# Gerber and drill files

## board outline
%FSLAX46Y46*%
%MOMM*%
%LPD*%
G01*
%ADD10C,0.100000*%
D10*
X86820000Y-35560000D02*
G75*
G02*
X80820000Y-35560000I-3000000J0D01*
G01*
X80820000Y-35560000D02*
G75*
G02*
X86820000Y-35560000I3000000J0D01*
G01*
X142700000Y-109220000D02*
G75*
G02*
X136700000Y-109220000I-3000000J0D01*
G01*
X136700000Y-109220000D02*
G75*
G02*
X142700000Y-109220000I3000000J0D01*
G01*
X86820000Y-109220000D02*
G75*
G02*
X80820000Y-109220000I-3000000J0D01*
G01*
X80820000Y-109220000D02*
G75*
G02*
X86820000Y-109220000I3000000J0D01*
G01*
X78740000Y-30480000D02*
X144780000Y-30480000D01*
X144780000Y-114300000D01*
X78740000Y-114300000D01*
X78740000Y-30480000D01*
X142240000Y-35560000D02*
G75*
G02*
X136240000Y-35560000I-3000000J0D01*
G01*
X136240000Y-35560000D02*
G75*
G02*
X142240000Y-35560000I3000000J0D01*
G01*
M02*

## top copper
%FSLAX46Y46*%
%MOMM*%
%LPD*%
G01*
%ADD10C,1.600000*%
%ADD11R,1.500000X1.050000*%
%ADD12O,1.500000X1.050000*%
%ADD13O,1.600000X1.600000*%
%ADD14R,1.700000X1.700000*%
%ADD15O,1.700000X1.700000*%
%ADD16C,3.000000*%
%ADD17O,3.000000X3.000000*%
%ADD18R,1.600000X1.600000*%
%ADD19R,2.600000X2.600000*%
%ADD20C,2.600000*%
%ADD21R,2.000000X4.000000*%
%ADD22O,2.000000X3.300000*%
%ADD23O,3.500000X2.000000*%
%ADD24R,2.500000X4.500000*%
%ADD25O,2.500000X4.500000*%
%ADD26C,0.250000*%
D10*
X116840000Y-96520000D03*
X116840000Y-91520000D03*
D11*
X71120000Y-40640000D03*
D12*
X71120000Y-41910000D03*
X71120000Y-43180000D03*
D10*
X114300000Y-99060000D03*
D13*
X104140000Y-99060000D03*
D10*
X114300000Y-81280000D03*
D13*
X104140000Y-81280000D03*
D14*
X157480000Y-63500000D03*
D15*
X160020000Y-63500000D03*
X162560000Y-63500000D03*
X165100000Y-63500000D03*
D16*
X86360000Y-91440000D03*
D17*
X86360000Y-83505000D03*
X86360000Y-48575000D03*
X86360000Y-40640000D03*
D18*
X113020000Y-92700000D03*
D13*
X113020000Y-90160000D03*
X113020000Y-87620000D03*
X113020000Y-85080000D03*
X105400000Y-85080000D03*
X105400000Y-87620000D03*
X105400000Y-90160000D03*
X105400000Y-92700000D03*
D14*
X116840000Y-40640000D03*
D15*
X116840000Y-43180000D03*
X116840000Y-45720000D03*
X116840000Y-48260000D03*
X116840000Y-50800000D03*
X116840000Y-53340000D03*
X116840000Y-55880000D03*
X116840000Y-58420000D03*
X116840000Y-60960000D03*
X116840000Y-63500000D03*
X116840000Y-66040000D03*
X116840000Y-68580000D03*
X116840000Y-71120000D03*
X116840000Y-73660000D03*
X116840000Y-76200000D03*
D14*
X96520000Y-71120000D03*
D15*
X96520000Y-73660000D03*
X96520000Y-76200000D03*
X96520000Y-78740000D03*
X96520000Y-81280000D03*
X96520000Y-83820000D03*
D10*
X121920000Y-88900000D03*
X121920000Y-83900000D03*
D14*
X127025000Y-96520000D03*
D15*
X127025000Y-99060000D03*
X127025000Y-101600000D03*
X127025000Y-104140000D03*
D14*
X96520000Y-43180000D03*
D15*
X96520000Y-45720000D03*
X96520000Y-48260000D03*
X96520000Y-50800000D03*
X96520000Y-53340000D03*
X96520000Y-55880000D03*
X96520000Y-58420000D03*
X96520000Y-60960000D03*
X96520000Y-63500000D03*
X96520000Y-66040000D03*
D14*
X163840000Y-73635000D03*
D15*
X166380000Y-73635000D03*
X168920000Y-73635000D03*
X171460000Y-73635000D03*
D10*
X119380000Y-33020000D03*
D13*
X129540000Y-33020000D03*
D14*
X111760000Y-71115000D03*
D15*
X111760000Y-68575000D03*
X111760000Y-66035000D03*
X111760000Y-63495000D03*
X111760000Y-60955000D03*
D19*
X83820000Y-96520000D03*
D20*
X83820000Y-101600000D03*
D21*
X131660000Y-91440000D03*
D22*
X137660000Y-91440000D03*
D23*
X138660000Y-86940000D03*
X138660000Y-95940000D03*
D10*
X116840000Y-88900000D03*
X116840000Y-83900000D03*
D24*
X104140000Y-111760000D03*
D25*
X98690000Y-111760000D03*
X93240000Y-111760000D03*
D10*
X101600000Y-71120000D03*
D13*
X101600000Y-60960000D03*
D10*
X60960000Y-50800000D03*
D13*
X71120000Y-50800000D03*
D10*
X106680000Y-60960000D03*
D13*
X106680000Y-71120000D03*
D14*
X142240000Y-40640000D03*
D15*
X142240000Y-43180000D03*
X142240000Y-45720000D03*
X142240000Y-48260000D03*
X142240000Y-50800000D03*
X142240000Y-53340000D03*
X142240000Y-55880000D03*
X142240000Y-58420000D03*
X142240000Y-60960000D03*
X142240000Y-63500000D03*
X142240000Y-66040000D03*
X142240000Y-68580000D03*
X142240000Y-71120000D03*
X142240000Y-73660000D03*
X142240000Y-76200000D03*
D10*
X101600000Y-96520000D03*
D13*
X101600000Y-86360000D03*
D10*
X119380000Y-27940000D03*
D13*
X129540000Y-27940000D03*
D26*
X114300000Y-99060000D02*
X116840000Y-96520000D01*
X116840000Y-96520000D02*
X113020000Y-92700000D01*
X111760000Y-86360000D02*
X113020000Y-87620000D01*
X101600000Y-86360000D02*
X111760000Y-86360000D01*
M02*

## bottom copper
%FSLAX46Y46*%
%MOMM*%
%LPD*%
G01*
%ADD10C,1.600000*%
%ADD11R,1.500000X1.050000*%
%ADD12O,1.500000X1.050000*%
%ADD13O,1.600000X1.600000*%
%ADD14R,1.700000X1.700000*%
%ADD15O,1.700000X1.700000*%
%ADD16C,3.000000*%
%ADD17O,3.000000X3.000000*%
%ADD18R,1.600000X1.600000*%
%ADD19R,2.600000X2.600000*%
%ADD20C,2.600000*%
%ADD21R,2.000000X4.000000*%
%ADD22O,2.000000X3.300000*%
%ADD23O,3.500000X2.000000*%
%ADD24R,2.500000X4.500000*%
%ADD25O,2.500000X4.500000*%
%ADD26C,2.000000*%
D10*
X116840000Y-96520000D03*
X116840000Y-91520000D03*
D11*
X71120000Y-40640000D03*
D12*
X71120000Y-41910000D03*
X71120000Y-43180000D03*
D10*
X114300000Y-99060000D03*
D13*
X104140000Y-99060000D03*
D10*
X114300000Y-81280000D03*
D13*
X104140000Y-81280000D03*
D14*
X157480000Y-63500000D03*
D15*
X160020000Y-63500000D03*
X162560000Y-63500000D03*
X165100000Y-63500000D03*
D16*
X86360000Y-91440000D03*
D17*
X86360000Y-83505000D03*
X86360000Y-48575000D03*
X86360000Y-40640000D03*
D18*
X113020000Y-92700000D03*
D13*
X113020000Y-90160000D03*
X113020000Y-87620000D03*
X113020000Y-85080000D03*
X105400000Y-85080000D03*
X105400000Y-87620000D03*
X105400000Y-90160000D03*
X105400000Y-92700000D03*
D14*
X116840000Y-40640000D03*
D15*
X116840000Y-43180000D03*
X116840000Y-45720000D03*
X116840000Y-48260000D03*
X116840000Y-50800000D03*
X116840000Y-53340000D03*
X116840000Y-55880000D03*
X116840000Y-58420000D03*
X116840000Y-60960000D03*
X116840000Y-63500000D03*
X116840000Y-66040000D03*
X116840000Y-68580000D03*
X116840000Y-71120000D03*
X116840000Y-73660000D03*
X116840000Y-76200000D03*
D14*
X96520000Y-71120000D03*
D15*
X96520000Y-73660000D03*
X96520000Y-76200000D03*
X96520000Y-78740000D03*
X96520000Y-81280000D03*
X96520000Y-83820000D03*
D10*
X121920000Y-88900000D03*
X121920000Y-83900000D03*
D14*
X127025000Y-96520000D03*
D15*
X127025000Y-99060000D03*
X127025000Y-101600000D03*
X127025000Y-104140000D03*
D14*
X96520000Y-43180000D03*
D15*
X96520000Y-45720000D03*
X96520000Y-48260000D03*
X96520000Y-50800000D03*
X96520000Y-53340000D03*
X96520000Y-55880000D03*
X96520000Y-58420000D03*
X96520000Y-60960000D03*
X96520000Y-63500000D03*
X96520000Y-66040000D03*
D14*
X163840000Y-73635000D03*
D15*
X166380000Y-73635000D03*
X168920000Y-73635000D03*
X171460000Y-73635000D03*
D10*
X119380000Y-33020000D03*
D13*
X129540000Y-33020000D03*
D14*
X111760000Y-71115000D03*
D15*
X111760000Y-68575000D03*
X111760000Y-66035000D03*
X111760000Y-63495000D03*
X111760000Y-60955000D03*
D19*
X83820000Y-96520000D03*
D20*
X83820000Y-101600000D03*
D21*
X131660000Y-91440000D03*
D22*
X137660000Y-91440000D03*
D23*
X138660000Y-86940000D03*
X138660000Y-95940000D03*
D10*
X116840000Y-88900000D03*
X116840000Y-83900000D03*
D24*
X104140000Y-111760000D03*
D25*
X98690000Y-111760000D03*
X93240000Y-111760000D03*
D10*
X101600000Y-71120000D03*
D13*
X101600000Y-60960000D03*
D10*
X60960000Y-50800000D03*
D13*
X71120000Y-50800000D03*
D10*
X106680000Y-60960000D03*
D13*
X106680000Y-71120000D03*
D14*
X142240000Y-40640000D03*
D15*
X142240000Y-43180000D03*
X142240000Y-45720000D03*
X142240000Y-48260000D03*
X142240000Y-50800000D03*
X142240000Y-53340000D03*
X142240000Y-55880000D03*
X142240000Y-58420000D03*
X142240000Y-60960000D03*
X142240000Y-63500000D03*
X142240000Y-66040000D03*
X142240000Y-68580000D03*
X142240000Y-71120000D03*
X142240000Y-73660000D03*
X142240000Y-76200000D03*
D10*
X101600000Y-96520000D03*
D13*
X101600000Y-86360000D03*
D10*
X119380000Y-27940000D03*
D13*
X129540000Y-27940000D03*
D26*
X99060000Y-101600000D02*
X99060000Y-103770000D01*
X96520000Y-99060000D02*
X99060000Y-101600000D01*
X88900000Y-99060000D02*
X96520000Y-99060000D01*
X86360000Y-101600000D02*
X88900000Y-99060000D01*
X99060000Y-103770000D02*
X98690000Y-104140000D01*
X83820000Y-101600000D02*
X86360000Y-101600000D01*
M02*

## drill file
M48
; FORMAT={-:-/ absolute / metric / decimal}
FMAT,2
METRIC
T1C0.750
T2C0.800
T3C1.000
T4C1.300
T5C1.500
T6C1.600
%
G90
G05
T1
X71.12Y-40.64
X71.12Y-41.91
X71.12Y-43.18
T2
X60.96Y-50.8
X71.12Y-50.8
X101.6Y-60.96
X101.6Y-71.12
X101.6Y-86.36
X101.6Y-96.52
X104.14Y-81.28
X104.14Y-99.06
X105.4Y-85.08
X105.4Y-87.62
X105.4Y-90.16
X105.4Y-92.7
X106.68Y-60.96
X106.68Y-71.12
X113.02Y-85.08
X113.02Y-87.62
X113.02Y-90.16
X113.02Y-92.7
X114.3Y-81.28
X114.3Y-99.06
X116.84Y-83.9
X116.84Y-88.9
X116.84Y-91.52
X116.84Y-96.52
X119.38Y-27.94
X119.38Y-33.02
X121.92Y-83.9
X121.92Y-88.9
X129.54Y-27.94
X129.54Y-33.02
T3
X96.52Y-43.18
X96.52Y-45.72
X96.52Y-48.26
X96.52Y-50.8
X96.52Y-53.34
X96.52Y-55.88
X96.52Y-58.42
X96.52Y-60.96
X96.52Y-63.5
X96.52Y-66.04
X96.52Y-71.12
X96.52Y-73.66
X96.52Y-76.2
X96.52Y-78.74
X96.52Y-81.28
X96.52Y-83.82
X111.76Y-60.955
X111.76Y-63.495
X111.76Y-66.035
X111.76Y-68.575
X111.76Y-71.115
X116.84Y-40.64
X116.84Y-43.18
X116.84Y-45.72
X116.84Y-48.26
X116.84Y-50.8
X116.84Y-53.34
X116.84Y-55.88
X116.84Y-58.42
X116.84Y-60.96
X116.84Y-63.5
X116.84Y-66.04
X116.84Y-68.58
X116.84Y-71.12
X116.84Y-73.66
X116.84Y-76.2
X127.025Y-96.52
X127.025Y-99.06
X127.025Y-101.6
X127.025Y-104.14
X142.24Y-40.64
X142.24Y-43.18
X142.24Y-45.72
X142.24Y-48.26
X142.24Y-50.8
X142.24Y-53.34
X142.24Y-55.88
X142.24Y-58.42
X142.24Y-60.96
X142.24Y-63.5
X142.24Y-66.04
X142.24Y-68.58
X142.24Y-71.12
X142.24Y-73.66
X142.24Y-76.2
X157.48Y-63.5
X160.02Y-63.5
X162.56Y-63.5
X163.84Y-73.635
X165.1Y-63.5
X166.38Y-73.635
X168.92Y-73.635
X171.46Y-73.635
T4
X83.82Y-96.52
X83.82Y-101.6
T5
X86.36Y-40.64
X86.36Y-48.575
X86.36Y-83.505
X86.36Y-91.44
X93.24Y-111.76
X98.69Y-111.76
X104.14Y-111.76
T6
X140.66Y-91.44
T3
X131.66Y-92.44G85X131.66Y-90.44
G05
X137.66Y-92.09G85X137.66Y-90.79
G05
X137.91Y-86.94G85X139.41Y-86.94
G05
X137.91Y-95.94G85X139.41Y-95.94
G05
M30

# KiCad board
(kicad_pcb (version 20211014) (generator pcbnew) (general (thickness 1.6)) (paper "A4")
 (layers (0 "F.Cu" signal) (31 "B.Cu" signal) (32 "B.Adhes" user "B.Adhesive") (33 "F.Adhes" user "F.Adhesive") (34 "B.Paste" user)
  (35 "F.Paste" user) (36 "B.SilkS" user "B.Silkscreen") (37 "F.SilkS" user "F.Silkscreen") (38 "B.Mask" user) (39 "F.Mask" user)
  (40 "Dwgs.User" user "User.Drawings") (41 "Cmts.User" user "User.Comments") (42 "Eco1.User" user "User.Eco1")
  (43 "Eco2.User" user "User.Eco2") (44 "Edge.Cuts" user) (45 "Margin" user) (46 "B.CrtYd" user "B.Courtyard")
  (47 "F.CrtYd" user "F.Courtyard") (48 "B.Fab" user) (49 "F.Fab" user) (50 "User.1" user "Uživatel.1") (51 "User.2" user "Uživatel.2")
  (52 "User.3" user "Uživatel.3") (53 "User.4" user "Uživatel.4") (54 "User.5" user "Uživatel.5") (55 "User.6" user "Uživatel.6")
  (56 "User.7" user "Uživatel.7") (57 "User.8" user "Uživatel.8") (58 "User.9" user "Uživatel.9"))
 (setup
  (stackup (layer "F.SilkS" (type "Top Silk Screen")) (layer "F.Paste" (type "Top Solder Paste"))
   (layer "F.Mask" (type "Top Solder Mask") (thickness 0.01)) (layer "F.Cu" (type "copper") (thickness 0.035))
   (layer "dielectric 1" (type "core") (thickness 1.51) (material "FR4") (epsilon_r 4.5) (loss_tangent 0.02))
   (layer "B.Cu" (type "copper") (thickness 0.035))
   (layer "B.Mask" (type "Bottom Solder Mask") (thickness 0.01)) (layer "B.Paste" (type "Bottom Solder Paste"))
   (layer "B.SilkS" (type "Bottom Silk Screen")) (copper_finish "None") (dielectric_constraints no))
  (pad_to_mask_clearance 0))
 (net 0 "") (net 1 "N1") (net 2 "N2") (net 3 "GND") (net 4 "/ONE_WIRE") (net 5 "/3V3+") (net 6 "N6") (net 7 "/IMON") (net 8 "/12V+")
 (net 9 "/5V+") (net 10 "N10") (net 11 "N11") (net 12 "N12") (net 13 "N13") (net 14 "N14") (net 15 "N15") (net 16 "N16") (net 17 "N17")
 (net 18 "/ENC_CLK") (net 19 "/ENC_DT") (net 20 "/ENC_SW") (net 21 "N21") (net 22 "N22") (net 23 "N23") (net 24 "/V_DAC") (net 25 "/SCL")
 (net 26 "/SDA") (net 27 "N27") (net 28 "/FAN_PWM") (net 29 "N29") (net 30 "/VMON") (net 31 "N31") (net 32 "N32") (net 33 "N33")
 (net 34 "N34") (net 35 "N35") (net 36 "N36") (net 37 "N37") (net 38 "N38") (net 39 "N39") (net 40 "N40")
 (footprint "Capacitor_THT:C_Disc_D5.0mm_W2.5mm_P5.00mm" (layer "F.Cu") (at 116.84 96.52 90)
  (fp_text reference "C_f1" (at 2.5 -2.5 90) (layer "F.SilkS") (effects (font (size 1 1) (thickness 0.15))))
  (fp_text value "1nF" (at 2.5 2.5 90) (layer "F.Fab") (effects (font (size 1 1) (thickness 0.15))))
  (pad "1" thru_hole circle locked (at 0 0 90) (size 1.6 1.6) (drill 0.8) (layers *.Cu *.Mask) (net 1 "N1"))
  (pad "2" thru_hole circle locked (at 5 0 90) (size 1.6 1.6) (drill 0.8) (layers *.Cu *.Mask) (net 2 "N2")))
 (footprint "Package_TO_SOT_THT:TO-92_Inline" (layer "F.Cu") (at 71.12 40.64 -90)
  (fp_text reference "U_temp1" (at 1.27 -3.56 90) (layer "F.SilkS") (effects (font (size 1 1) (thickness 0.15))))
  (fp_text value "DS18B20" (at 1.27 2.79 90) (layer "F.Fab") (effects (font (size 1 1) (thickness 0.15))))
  (pad "1" thru_hole rect locked (at 0 0 270) (size 1.05 1.5) (drill 0.75) (layers *.Cu *.Mask) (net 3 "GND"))
  (pad "2" thru_hole oval locked (at 1.27 0 270) (size 1.05 1.5) (drill 0.75) (layers *.Cu *.Mask) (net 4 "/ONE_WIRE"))
  (pad "3" thru_hole oval locked (at 2.54 0 270) (size 1.05 1.5) (drill 0.75) (layers *.Cu *.Mask) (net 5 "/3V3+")))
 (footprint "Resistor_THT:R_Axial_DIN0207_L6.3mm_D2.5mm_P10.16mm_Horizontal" (layer "F.Cu") (at 114.3 99.06 180)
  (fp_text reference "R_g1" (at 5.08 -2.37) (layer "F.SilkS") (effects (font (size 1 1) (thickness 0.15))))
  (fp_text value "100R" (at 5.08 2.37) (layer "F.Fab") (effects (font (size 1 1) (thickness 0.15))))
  (pad "1" thru_hole circle locked (at 0 0 180) (size 1.6 1.6) (drill 0.8) (layers *.Cu *.Mask) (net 1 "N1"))
  (pad "2" thru_hole oval locked (at 10.16 0 180) (size 1.6 1.6) (drill 0.8) (layers *.Cu *.Mask) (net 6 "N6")))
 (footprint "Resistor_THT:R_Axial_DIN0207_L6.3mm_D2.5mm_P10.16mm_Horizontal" (layer "F.Cu") (at 114.3 81.28 180)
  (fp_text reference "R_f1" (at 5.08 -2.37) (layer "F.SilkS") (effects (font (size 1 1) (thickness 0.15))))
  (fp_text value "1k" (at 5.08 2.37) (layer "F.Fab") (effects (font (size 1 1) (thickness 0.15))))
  (pad "1" thru_hole circle locked (at 0 0 180) (size 1.6 1.6) (drill 0.8) (layers *.Cu *.Mask) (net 2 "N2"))
  (pad "2" thru_hole oval locked (at 10.16 0 180) (size 1.6 1.6) (drill 0.8) (layers *.Cu *.Mask) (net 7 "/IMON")))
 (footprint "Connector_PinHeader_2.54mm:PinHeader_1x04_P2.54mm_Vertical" (layer "F.Cu") (at 157.48 63.5 90)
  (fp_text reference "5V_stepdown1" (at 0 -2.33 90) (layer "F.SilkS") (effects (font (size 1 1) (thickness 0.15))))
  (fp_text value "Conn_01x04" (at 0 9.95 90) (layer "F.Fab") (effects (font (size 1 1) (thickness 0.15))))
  (pad "1" thru_hole rect locked (at 0 0 90) (size 1.7 1.7) (drill 1) (layers *.Cu *.Mask) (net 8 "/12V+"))
  (pad "2" thru_hole oval locked (at 0 2.54 90) (size 1.7 1.7) (drill 1) (layers *.Cu *.Mask) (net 3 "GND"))
  (pad "3" thru_hole oval locked (at 0 5.08 90) (size 1.7 1.7) (drill 1) (layers *.Cu *.Mask) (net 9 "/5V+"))
  (pad "4" thru_hole oval locked (at 0 7.62 90) (size 1.7 1.7) (drill 1) (layers *.Cu *.Mask) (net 3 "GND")))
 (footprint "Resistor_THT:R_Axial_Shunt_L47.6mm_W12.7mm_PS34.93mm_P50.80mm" (layer "F.Cu") (at 86.36 91.44 90)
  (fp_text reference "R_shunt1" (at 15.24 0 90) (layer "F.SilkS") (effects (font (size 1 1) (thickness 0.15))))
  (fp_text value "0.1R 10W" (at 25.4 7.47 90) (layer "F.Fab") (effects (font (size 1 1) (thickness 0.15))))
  (pad "1" thru_hole circle locked (at 0 0 90) (size 3 3) (drill 1.5) (layers *.Cu *.Mask) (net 3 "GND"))
  (pad "2" thru_hole oval locked (at 7.935 0 90) (size 3 3) (drill 1.5) (layers *.Cu *.Mask) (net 7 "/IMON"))
  (pad "3" thru_hole oval locked (at 42.865 0 90) (size 3 3) (drill 1.5) (layers *.Cu *.Mask))
  (pad "4" thru_hole oval locked (at 50.8 0 90) (size 3 3) (drill 1.5) (layers *.Cu *.Mask)))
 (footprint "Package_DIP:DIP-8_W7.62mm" (layer "F.Cu") (at 113.02 92.7 180)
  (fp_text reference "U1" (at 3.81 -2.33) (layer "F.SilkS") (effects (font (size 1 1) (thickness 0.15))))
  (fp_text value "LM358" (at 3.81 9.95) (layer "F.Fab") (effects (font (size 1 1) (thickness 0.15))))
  (pad "1" thru_hole rect locked (at 0 0 180) (size 1.6 1.6) (drill 0.8) (layers *.Cu *.Mask) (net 1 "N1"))
  (pad "2" thru_hole oval locked (at 0 2.54 180) (size 1.6 1.6) (drill 0.8) (layers *.Cu *.Mask) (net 2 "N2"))
  (pad "3" thru_hole oval locked (at 0 5.08 180) (size 1.6 1.6) (drill 0.8) (layers *.Cu *.Mask) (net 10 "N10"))
  (pad "4" thru_hole oval locked (at 0 7.62 180) (size 1.6 1.6) (drill 0.8) (layers *.Cu *.Mask) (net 3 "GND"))
  (pad "5" thru_hole oval locked (at 7.62 7.62 180) (size 1.6 1.6) (drill 0.8) (layers *.Cu *.Mask))
  (pad "6" thru_hole oval locked (at 7.62 5.08 180) (size 1.6 1.6) (drill 0.8) (layers *.Cu *.Mask))
  (pad "7" thru_hole oval locked (at 7.62 2.54 180) (size 1.6 1.6) (drill 0.8) (layers *.Cu *.Mask))
  (pad "8" thru_hole oval locked (at 7.62 0 180) (size 1.6 1.6) (drill 0.8) (layers *.Cu *.Mask) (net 8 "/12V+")))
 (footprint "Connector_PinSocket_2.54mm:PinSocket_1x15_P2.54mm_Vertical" (layer "F.Cu") (at 116.84 40.64)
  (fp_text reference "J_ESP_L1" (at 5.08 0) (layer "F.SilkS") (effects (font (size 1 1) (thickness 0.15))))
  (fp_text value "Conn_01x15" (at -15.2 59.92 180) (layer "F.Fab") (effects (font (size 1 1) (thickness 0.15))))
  (pad "1" thru_hole rect locked (at 0 0) (size 1.7 1.7) (drill 1) (layers *.Cu *.Mask) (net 5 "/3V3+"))
  (pad "2" thru_hole oval locked (at 0 2.54) (size 1.7 1.7) (drill 1) (layers *.Cu *.Mask) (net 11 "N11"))
  (pad "3" thru_hole oval locked (at 0 5.08) (size 1.7 1.7) (drill 1) (layers *.Cu *.Mask) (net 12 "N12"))
  (pad "4" thru_hole oval locked (at 0 7.62) (size 1.7 1.7) (drill 1) (layers *.Cu *.Mask) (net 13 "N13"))
  (pad "5" thru_hole oval locked (at 0 10.16) (size 1.7 1.7) (drill 1) (layers *.Cu *.Mask) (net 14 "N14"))
  (pad "6" thru_hole oval locked (at 0 12.7) (size 1.7 1.7) (drill 1) (layers *.Cu *.Mask) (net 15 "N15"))
  (pad "7" thru_hole oval locked (at 0 15.24) (size 1.7 1.7) (drill 1) (layers *.Cu *.Mask) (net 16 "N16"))
  (pad "8" thru_hole oval locked (at 0 17.78) (size 1.7 1.7) (drill 1) (layers *.Cu *.Mask) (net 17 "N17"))
  (pad "9" thru_hole oval locked (at 0 20.32) (size 1.7 1.7) (drill 1) (layers *.Cu *.Mask) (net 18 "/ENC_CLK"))
  (pad "10" thru_hole oval locked (at 0 22.86) (size 1.7 1.7) (drill 1) (layers *.Cu *.Mask) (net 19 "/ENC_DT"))
  (pad "11" thru_hole oval locked (at 0 25.4) (size 1.7 1.7) (drill 1) (layers *.Cu *.Mask) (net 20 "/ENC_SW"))
  (pad "12" thru_hole oval locked (at 0 27.94) (size 1.7 1.7) (drill 1) (layers *.Cu *.Mask) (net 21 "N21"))
  (pad "13" thru_hole oval locked (at 0 30.48) (size 1.7 1.7) (drill 1) (layers *.Cu *.Mask) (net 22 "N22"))
  (pad "14" thru_hole oval locked (at 0 33.02) (size 1.7 1.7) (drill 1) (layers *.Cu *.Mask) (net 3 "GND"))
  (pad "15" thru_hole oval locked (at 0 35.56) (size 1.7 1.7) (drill 1) (layers *.Cu *.Mask) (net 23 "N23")))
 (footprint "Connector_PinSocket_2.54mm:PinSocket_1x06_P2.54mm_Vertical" (layer "F.Cu") (at 96.52 71.12)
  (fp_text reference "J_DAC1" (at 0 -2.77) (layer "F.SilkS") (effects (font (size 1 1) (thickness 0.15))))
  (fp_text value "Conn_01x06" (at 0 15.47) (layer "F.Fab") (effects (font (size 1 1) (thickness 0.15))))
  (pad "1" thru_hole rect locked (at 0 0) (size 1.7 1.7) (drill 1) (layers *.Cu *.Mask) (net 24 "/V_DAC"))
  (pad "2" thru_hole oval locked (at 0 2.54) (size 1.7 1.7) (drill 1) (layers *.Cu *.Mask) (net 3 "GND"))
  (pad "3" thru_hole oval locked (at 0 5.08) (size 1.7 1.7) (drill 1) (layers *.Cu *.Mask) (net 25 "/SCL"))
  (pad "4" thru_hole oval locked (at 0 7.62) (size 1.7 1.7) (drill 1) (layers *.Cu *.Mask) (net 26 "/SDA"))
  (pad "5" thru_hole oval locked (at 0 10.16) (size 1.7 1.7) (drill 1) (layers *.Cu *.Mask) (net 5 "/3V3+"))
  (pad "6" thru_hole oval locked (at 0 12.7) (size 1.7 1.7) (drill 1) (layers *.Cu *.Mask) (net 3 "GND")))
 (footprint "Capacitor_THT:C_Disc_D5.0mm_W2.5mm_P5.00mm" (layer "F.Cu") (at 121.92 88.9 90)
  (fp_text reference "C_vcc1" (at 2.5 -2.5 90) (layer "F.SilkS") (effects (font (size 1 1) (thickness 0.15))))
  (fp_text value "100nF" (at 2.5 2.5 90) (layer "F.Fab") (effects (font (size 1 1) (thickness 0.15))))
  (pad "1" thru_hole circle locked (at 0 0 90) (size 1.6 1.6) (drill 0.8) (layers *.Cu *.Mask) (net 8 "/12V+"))
  (pad "2" thru_hole circle locked (at 5 0 90) (size 1.6 1.6) (drill 0.8) (layers *.Cu *.Mask) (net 3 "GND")))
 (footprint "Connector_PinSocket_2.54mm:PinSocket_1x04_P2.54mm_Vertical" (layer "F.Cu") (at 127.025 96.52)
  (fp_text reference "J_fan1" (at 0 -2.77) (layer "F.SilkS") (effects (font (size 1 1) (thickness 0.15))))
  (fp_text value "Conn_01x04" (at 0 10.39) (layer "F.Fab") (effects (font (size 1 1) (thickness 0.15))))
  (pad "1" thru_hole rect locked (at 0 0) (size 1.7 1.7) (drill 1) (layers *.Cu *.Mask) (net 3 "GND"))
  (pad "2" thru_hole oval locked (at 0 2.54) (size 1.7 1.7) (drill 1) (layers *.Cu *.Mask) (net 8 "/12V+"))
  (pad "3" thru_hole oval locked (at 0 5.08) (size 1.7 1.7) (drill 1) (layers *.Cu *.Mask) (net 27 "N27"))
  (pad "4" thru_hole oval locked (at 0 7.62) (size 1.7 1.7) (drill 1) (layers *.Cu *.Mask) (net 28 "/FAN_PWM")))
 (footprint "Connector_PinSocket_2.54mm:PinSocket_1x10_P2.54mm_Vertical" (layer "F.Cu") (at 96.52 43.18)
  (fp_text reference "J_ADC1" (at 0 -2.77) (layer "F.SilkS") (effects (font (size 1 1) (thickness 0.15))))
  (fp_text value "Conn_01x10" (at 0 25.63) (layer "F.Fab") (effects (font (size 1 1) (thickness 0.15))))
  (pad "1" thru_hole rect locked (at 0 0) (size 1.7 1.7) (drill 1) (layers *.Cu *.Mask) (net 5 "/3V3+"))
  (pad "2" thru_hole oval locked (at 0 2.54) (size 1.7 1.7) (drill 1) (layers *.Cu *.Mask) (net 3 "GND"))
  (pad "3" thru_hole oval locked (at 0 5.08) (size 1.7 1.7) (drill 1) (layers *.Cu *.Mask) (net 25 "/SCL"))
  (pad "4" thru_hole oval locked (at 0 7.62) (size 1.7 1.7) (drill 1) (layers *.Cu *.Mask) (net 26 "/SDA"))
  (pad "5" thru_hole oval locked (at 0 10.16) (size 1.7 1.7) (drill 1) (layers *.Cu *.Mask) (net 3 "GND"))
  (pad "6" thru_hole oval locked (at 0 12.7) (size 1.7 1.7) (drill 1) (layers *.Cu *.Mask) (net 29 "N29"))
  (pad "7" thru_hole oval locked (at 0 15.24) (size 1.7 1.7) (drill 1) (layers *.Cu *.Mask) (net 7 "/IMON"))
  (pad "8" thru_hole oval locked (at 0 17.78) (size 1.7 1.7) (drill 1) (layers *.Cu *.Mask) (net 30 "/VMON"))
  (pad "9" thru_hole oval locked (at 0 20.32) (size 1.7 1.7) (drill 1) (layers *.Cu *.Mask) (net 3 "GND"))
  (pad "10" thru_hole oval locked (at 0 22.86) (size 1.7 1.7) (drill 1) (layers *.Cu *.Mask) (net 3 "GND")))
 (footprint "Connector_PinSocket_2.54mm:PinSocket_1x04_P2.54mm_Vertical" (layer "F.Cu") (at 163.84 73.635 90)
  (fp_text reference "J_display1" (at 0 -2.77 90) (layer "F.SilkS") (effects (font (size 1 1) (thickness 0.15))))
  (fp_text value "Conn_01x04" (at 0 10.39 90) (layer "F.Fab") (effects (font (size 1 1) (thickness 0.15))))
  (pad "1" thru_hole rect locked (at 0 0 90) (size 1.7 1.7) (drill 1) (layers *.Cu *.Mask) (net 3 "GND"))
  (pad "2" thru_hole oval locked (at 0 2.54 90) (size 1.7 1.7) (drill 1) (layers *.Cu *.Mask) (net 5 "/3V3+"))
  (pad "3" thru_hole oval locked (at 0 5.08 90) (size 1.7 1.7) (drill 1) (layers *.Cu *.Mask) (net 25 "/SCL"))
  (pad "4" thru_hole oval locked (at 0 7.62 90) (size 1.7 1.7) (drill 1) (layers *.Cu *.Mask) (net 26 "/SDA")))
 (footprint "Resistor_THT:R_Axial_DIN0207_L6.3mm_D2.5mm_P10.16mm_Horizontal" (layer "F.Cu") (at 119.38 33.02)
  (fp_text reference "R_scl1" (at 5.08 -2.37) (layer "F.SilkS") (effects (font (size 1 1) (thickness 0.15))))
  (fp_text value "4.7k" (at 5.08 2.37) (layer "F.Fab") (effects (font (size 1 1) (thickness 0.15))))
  (pad "1" thru_hole circle locked (at 0 0) (size 1.6 1.6) (drill 0.8) (layers *.Cu *.Mask) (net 5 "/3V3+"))
  (pad "2" thru_hole oval locked (at 10.16 0) (size 1.6 1.6) (drill 0.8) (layers *.Cu *.Mask) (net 25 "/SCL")))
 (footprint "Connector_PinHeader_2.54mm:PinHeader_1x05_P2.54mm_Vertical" (layer "F.Cu") (at 111.76 71.115 180)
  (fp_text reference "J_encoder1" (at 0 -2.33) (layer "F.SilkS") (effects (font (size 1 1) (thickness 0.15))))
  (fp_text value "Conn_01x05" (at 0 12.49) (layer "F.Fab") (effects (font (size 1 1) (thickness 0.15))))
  (pad "1" thru_hole rect locked (at 0 0 180) (size 1.7 1.7) (drill 1) (layers *.Cu *.Mask) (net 3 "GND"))
  (pad "2" thru_hole oval locked (at 0 2.54 180) (size 1.7 1.7) (drill 1) (layers *.Cu *.Mask) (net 5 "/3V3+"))
  (pad "3" thru_hole oval locked (at 0 5.08 180) (size 1.7 1.7) (drill 1) (layers *.Cu *.Mask) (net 20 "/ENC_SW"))
  (pad "4" thru_hole oval locked (at 0 7.62 180) (size 1.7 1.7) (drill 1) (layers *.Cu *.Mask) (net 19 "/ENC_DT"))
  (pad "5" thru_hole oval locked (at 0 10.16 180) (size 1.7 1.7) (drill 1) (layers *.Cu *.Mask) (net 18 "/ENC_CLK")))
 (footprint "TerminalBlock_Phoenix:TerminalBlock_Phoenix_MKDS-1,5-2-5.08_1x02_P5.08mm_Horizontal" (layer "F.Cu") (at 83.82 96.52 -90)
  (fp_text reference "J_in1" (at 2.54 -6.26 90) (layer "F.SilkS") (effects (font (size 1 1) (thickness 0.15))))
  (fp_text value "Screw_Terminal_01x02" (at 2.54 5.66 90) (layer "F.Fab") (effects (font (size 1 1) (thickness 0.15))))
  (pad "1" thru_hole rect locked (at 0 0 270) (size 2.6 2.6) (drill 1.3) (layers *.Cu *.Mask) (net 3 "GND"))
  (pad "2" thru_hole circle locked (at 5.08 0 270) (size 2.6 2.6) (drill 1.3) (layers *.Cu *.Mask) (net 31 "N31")))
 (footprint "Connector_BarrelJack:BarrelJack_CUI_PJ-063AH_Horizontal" (layer "F.Cu") (at 131.66 91.44 90)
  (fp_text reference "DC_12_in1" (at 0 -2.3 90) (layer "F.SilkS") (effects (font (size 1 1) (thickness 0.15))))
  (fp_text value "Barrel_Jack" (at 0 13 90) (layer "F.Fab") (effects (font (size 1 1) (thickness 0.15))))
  (pad "" np_thru_hole circle locked (at 0 9 90) (size 1.6 1.6) (drill 1.6) (layers *.Cu *.Mask))
  (pad "1" thru_hole rect locked (at 0 0 90) (size 4 2) (drill oval 3 1) (layers *.Cu *.Mask) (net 8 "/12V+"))
  (pad "2" thru_hole oval locked (at 0 6 90) (size 3.3 2) (drill oval 2.3 1) (layers *.Cu *.Mask) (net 3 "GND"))
  (pad "MP" thru_hole oval locked (at 4.5 7 90) (size 2 3.5) (drill oval 1 2.5) (layers *.Cu *.Mask))
  (pad "MP" thru_hole oval locked (at -4.5 7 90) (size 2 3.5) (drill oval 1 2.5) (layers *.Cu *.Mask)))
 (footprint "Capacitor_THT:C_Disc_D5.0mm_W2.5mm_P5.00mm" (layer "F.Cu") (at 116.84 88.9 90)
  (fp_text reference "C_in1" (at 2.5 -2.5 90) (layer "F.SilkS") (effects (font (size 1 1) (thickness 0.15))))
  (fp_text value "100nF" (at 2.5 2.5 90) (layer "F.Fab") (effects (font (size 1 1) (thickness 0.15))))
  (pad "1" thru_hole circle locked (at 0 0 90) (size 1.6 1.6) (drill 0.8) (layers *.Cu *.Mask) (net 10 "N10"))
  (pad "2" thru_hole circle locked (at 5 0 90) (size 1.6 1.6) (drill 0.8) (layers *.Cu *.Mask) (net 3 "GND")))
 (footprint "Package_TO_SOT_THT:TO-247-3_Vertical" (layer "F.Cu") (at 104.14 111.76 180)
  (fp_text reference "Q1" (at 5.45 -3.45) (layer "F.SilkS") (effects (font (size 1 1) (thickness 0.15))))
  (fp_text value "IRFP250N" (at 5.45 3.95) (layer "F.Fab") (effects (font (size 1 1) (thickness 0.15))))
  (pad "1" thru_hole rect locked (at 0 0 180) (size 2.5 4.5) (drill 1.5) (layers *.Cu *.Mask) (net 6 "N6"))
  (pad "2" thru_hole oval locked (at 5.45 0 180) (size 2.5 4.5) (drill 1.5) (layers *.Cu *.Mask) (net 31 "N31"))
  (pad "3" thru_hole oval locked (at 10.9 0 180) (size 2.5 4.5) (drill 1.5) (layers *.Cu *.Mask) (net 7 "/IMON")))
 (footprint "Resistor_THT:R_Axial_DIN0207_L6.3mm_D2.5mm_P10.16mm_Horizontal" (layer "F.Cu") (at 101.6 71.12 90)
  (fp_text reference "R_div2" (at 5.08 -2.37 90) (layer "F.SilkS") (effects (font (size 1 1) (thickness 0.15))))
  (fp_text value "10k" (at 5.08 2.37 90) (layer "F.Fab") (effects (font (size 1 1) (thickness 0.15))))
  (pad "1" thru_hole circle locked (at 0 0 90) (size 1.6 1.6) (drill 0.8) (layers *.Cu *.Mask) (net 3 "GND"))
  (pad "2" thru_hole oval locked (at 10.16 0 90) (size 1.6 1.6) (drill 0.8) (layers *.Cu *.Mask) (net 30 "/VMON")))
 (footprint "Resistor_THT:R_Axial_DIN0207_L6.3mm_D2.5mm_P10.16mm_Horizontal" (layer "F.Cu") (at 60.96 50.8)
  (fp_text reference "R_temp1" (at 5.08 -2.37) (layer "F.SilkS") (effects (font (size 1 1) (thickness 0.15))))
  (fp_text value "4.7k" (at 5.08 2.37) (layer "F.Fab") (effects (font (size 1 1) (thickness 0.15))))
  (pad "1" thru_hole circle locked (at 0 0) (size 1.6 1.6) (drill 0.8) (layers *.Cu *.Mask) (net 4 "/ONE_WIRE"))
  (pad "2" thru_hole oval locked (at 10.16 0) (size 1.6 1.6) (drill 0.8) (layers *.Cu *.Mask) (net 5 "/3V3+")))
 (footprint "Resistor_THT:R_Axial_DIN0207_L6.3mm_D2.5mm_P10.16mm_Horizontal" (layer "F.Cu") (at 106.68 60.96 -90)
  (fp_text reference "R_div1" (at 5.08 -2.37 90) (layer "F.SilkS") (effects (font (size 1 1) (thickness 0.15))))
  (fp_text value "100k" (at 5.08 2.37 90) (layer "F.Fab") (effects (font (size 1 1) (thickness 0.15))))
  (pad "1" thru_hole circle locked (at 0 0 270) (size 1.6 1.6) (drill 0.8) (layers *.Cu *.Mask) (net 30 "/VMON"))
  (pad "2" thru_hole oval locked (at 10.16 0 270) (size 1.6 1.6) (drill 0.8) (layers *.Cu *.Mask) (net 31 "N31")))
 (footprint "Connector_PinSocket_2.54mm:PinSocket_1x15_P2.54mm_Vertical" (layer "F.Cu") (at 142.24 40.64)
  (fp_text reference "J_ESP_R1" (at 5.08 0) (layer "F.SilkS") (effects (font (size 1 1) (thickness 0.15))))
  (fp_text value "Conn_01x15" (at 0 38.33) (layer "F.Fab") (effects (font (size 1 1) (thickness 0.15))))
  (pad "1" thru_hole rect locked (at 0 0) (size 1.7 1.7) (drill 1) (layers *.Cu *.Mask) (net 9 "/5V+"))
  (pad "2" thru_hole oval locked (at 0 2.54) (size 1.7 1.7) (drill 1) (layers *.Cu *.Mask) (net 3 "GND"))
  (pad "3" thru_hole oval locked (at 0 5.08) (size 1.7 1.7) (drill 1) (layers *.Cu *.Mask) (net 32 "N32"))
  (pad "4" thru_hole oval locked (at 0 7.62) (size 1.7 1.7) (drill 1) (layers *.Cu *.Mask) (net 25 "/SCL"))
  (pad "5" thru_hole oval locked (at 0 10.16) (size 1.7 1.7) (drill 1) (layers *.Cu *.Mask) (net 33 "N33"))
  (pad "6" thru_hole oval locked (at 0 12.7) (size 1.7 1.7) (drill 1) (layers *.Cu *.Mask) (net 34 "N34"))
  (pad "7" thru_hole oval locked (at 0 15.24) (size 1.7 1.7) (drill 1) (layers *.Cu *.Mask) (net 26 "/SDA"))
  (pad "8" thru_hole oval locked (at 0 17.78) (size 1.7 1.7) (drill 1) (layers *.Cu *.Mask) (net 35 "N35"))
  (pad "9" thru_hole oval locked (at 0 20.32) (size 1.7 1.7) (drill 1) (layers *.Cu *.Mask) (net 28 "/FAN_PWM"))
  (pad "10" thru_hole oval locked (at 0 22.86) (size 1.7 1.7) (drill 1) (layers *.Cu *.Mask) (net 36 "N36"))
  (pad "11" thru_hole oval locked (at 0 25.4) (size 1.7 1.7) (drill 1) (layers *.Cu *.Mask) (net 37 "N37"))
  (pad "12" thru_hole oval locked (at 0 27.94) (size 1.7 1.7) (drill 1) (layers *.Cu *.Mask) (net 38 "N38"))
  (pad "13" thru_hole oval locked (at 0 30.48) (size 1.7 1.7) (drill 1) (layers *.Cu *.Mask) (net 4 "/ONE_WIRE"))
  (pad "14" thru_hole oval locked (at 0 33.02) (size 1.7 1.7) (drill 1) (layers *.Cu *.Mask) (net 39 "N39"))
  (pad "15" thru_hole oval locked (at 0 35.56) (size 1.7 1.7) (drill 1) (layers *.Cu *.Mask) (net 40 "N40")))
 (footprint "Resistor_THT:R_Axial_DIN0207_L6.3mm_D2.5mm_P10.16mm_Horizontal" (layer "F.Cu") (at 101.6 96.52 90)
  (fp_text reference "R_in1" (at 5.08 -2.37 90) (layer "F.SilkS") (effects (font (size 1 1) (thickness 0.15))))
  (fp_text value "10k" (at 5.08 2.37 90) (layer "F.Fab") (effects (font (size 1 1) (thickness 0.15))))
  (pad "1" thru_hole circle locked (at 0 0 90) (size 1.6 1.6) (drill 0.8) (layers *.Cu *.Mask) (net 24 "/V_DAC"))
  (pad "2" thru_hole oval locked (at 10.16 0 90) (size 1.6 1.6) (drill 0.8) (layers *.Cu *.Mask) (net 10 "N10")))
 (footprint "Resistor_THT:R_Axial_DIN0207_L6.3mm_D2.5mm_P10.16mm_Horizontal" (layer "F.Cu") (at 119.38 27.94)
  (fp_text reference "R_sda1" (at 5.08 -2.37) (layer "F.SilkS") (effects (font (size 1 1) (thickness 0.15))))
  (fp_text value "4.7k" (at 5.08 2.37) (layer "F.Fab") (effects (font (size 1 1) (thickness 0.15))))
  (pad "1" thru_hole circle locked (at 0 0) (size 1.6 1.6) (drill 0.8) (layers *.Cu *.Mask) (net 5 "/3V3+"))
  (pad "2" thru_hole oval locked (at 10.16 0) (size 1.6 1.6) (drill 0.8) (layers *.Cu *.Mask) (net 26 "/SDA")))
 (gr_circle (center 83.82 35.56) (end 86.82 35.56) (layer "Edge.Cuts") (width 0.1) (fill none))
 (gr_circle (center 139.7 109.22) (end 142.7 109.22) (layer "Edge.Cuts") (width 0.1) (fill none))
 (gr_circle (center 83.82 109.22) (end 86.82 109.22) (layer "Edge.Cuts") (width 0.1) (fill none))
 (gr_rect (start 78.74 30.48) (end 144.78 114.3) (layer "Edge.Cuts") (width 0.1) (fill none))
 (gr_circle (center 139.24 35.56) (end 142.24 35.56) (layer "Edge.Cuts") (width 0.1) (fill none))
 (segment (start 114.3 99.06) (end 116.84 96.52) (width 0.25) (layer "F.Cu") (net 1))
 (segment (start 116.84 96.52) (end 113.02 92.7) (width 0.25) (layer "F.Cu") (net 1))
 (segment (start 111.76 86.36) (end 113.02 87.62) (width 0.25) (layer "F.Cu") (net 10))
 (segment (start 101.6 86.36) (end 111.76 86.36) (width 0.25) (layer "F.Cu") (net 10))
 (segment (start 99.06 101.6) (end 99.06 103.77) (width 2) (layer "B.Cu") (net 31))
 (segment (start 96.52 99.06) (end 99.06 101.6) (width 2) (layer "B.Cu") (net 31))
 (segment (start 88.9 99.06) (end 96.52 99.06) (width 2) (layer "B.Cu") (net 31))
 (segment (start 86.36 101.6) (end 88.9 99.06) (width 2) (layer "B.Cu") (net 31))
 (segment (start 99.06 103.77) (end 98.69 104.14) (width 2) (layer "B.Cu") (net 31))
 (segment (start 83.82 101.6) (end 86.36 101.6) (width 2) (layer "B.Cu") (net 31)))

